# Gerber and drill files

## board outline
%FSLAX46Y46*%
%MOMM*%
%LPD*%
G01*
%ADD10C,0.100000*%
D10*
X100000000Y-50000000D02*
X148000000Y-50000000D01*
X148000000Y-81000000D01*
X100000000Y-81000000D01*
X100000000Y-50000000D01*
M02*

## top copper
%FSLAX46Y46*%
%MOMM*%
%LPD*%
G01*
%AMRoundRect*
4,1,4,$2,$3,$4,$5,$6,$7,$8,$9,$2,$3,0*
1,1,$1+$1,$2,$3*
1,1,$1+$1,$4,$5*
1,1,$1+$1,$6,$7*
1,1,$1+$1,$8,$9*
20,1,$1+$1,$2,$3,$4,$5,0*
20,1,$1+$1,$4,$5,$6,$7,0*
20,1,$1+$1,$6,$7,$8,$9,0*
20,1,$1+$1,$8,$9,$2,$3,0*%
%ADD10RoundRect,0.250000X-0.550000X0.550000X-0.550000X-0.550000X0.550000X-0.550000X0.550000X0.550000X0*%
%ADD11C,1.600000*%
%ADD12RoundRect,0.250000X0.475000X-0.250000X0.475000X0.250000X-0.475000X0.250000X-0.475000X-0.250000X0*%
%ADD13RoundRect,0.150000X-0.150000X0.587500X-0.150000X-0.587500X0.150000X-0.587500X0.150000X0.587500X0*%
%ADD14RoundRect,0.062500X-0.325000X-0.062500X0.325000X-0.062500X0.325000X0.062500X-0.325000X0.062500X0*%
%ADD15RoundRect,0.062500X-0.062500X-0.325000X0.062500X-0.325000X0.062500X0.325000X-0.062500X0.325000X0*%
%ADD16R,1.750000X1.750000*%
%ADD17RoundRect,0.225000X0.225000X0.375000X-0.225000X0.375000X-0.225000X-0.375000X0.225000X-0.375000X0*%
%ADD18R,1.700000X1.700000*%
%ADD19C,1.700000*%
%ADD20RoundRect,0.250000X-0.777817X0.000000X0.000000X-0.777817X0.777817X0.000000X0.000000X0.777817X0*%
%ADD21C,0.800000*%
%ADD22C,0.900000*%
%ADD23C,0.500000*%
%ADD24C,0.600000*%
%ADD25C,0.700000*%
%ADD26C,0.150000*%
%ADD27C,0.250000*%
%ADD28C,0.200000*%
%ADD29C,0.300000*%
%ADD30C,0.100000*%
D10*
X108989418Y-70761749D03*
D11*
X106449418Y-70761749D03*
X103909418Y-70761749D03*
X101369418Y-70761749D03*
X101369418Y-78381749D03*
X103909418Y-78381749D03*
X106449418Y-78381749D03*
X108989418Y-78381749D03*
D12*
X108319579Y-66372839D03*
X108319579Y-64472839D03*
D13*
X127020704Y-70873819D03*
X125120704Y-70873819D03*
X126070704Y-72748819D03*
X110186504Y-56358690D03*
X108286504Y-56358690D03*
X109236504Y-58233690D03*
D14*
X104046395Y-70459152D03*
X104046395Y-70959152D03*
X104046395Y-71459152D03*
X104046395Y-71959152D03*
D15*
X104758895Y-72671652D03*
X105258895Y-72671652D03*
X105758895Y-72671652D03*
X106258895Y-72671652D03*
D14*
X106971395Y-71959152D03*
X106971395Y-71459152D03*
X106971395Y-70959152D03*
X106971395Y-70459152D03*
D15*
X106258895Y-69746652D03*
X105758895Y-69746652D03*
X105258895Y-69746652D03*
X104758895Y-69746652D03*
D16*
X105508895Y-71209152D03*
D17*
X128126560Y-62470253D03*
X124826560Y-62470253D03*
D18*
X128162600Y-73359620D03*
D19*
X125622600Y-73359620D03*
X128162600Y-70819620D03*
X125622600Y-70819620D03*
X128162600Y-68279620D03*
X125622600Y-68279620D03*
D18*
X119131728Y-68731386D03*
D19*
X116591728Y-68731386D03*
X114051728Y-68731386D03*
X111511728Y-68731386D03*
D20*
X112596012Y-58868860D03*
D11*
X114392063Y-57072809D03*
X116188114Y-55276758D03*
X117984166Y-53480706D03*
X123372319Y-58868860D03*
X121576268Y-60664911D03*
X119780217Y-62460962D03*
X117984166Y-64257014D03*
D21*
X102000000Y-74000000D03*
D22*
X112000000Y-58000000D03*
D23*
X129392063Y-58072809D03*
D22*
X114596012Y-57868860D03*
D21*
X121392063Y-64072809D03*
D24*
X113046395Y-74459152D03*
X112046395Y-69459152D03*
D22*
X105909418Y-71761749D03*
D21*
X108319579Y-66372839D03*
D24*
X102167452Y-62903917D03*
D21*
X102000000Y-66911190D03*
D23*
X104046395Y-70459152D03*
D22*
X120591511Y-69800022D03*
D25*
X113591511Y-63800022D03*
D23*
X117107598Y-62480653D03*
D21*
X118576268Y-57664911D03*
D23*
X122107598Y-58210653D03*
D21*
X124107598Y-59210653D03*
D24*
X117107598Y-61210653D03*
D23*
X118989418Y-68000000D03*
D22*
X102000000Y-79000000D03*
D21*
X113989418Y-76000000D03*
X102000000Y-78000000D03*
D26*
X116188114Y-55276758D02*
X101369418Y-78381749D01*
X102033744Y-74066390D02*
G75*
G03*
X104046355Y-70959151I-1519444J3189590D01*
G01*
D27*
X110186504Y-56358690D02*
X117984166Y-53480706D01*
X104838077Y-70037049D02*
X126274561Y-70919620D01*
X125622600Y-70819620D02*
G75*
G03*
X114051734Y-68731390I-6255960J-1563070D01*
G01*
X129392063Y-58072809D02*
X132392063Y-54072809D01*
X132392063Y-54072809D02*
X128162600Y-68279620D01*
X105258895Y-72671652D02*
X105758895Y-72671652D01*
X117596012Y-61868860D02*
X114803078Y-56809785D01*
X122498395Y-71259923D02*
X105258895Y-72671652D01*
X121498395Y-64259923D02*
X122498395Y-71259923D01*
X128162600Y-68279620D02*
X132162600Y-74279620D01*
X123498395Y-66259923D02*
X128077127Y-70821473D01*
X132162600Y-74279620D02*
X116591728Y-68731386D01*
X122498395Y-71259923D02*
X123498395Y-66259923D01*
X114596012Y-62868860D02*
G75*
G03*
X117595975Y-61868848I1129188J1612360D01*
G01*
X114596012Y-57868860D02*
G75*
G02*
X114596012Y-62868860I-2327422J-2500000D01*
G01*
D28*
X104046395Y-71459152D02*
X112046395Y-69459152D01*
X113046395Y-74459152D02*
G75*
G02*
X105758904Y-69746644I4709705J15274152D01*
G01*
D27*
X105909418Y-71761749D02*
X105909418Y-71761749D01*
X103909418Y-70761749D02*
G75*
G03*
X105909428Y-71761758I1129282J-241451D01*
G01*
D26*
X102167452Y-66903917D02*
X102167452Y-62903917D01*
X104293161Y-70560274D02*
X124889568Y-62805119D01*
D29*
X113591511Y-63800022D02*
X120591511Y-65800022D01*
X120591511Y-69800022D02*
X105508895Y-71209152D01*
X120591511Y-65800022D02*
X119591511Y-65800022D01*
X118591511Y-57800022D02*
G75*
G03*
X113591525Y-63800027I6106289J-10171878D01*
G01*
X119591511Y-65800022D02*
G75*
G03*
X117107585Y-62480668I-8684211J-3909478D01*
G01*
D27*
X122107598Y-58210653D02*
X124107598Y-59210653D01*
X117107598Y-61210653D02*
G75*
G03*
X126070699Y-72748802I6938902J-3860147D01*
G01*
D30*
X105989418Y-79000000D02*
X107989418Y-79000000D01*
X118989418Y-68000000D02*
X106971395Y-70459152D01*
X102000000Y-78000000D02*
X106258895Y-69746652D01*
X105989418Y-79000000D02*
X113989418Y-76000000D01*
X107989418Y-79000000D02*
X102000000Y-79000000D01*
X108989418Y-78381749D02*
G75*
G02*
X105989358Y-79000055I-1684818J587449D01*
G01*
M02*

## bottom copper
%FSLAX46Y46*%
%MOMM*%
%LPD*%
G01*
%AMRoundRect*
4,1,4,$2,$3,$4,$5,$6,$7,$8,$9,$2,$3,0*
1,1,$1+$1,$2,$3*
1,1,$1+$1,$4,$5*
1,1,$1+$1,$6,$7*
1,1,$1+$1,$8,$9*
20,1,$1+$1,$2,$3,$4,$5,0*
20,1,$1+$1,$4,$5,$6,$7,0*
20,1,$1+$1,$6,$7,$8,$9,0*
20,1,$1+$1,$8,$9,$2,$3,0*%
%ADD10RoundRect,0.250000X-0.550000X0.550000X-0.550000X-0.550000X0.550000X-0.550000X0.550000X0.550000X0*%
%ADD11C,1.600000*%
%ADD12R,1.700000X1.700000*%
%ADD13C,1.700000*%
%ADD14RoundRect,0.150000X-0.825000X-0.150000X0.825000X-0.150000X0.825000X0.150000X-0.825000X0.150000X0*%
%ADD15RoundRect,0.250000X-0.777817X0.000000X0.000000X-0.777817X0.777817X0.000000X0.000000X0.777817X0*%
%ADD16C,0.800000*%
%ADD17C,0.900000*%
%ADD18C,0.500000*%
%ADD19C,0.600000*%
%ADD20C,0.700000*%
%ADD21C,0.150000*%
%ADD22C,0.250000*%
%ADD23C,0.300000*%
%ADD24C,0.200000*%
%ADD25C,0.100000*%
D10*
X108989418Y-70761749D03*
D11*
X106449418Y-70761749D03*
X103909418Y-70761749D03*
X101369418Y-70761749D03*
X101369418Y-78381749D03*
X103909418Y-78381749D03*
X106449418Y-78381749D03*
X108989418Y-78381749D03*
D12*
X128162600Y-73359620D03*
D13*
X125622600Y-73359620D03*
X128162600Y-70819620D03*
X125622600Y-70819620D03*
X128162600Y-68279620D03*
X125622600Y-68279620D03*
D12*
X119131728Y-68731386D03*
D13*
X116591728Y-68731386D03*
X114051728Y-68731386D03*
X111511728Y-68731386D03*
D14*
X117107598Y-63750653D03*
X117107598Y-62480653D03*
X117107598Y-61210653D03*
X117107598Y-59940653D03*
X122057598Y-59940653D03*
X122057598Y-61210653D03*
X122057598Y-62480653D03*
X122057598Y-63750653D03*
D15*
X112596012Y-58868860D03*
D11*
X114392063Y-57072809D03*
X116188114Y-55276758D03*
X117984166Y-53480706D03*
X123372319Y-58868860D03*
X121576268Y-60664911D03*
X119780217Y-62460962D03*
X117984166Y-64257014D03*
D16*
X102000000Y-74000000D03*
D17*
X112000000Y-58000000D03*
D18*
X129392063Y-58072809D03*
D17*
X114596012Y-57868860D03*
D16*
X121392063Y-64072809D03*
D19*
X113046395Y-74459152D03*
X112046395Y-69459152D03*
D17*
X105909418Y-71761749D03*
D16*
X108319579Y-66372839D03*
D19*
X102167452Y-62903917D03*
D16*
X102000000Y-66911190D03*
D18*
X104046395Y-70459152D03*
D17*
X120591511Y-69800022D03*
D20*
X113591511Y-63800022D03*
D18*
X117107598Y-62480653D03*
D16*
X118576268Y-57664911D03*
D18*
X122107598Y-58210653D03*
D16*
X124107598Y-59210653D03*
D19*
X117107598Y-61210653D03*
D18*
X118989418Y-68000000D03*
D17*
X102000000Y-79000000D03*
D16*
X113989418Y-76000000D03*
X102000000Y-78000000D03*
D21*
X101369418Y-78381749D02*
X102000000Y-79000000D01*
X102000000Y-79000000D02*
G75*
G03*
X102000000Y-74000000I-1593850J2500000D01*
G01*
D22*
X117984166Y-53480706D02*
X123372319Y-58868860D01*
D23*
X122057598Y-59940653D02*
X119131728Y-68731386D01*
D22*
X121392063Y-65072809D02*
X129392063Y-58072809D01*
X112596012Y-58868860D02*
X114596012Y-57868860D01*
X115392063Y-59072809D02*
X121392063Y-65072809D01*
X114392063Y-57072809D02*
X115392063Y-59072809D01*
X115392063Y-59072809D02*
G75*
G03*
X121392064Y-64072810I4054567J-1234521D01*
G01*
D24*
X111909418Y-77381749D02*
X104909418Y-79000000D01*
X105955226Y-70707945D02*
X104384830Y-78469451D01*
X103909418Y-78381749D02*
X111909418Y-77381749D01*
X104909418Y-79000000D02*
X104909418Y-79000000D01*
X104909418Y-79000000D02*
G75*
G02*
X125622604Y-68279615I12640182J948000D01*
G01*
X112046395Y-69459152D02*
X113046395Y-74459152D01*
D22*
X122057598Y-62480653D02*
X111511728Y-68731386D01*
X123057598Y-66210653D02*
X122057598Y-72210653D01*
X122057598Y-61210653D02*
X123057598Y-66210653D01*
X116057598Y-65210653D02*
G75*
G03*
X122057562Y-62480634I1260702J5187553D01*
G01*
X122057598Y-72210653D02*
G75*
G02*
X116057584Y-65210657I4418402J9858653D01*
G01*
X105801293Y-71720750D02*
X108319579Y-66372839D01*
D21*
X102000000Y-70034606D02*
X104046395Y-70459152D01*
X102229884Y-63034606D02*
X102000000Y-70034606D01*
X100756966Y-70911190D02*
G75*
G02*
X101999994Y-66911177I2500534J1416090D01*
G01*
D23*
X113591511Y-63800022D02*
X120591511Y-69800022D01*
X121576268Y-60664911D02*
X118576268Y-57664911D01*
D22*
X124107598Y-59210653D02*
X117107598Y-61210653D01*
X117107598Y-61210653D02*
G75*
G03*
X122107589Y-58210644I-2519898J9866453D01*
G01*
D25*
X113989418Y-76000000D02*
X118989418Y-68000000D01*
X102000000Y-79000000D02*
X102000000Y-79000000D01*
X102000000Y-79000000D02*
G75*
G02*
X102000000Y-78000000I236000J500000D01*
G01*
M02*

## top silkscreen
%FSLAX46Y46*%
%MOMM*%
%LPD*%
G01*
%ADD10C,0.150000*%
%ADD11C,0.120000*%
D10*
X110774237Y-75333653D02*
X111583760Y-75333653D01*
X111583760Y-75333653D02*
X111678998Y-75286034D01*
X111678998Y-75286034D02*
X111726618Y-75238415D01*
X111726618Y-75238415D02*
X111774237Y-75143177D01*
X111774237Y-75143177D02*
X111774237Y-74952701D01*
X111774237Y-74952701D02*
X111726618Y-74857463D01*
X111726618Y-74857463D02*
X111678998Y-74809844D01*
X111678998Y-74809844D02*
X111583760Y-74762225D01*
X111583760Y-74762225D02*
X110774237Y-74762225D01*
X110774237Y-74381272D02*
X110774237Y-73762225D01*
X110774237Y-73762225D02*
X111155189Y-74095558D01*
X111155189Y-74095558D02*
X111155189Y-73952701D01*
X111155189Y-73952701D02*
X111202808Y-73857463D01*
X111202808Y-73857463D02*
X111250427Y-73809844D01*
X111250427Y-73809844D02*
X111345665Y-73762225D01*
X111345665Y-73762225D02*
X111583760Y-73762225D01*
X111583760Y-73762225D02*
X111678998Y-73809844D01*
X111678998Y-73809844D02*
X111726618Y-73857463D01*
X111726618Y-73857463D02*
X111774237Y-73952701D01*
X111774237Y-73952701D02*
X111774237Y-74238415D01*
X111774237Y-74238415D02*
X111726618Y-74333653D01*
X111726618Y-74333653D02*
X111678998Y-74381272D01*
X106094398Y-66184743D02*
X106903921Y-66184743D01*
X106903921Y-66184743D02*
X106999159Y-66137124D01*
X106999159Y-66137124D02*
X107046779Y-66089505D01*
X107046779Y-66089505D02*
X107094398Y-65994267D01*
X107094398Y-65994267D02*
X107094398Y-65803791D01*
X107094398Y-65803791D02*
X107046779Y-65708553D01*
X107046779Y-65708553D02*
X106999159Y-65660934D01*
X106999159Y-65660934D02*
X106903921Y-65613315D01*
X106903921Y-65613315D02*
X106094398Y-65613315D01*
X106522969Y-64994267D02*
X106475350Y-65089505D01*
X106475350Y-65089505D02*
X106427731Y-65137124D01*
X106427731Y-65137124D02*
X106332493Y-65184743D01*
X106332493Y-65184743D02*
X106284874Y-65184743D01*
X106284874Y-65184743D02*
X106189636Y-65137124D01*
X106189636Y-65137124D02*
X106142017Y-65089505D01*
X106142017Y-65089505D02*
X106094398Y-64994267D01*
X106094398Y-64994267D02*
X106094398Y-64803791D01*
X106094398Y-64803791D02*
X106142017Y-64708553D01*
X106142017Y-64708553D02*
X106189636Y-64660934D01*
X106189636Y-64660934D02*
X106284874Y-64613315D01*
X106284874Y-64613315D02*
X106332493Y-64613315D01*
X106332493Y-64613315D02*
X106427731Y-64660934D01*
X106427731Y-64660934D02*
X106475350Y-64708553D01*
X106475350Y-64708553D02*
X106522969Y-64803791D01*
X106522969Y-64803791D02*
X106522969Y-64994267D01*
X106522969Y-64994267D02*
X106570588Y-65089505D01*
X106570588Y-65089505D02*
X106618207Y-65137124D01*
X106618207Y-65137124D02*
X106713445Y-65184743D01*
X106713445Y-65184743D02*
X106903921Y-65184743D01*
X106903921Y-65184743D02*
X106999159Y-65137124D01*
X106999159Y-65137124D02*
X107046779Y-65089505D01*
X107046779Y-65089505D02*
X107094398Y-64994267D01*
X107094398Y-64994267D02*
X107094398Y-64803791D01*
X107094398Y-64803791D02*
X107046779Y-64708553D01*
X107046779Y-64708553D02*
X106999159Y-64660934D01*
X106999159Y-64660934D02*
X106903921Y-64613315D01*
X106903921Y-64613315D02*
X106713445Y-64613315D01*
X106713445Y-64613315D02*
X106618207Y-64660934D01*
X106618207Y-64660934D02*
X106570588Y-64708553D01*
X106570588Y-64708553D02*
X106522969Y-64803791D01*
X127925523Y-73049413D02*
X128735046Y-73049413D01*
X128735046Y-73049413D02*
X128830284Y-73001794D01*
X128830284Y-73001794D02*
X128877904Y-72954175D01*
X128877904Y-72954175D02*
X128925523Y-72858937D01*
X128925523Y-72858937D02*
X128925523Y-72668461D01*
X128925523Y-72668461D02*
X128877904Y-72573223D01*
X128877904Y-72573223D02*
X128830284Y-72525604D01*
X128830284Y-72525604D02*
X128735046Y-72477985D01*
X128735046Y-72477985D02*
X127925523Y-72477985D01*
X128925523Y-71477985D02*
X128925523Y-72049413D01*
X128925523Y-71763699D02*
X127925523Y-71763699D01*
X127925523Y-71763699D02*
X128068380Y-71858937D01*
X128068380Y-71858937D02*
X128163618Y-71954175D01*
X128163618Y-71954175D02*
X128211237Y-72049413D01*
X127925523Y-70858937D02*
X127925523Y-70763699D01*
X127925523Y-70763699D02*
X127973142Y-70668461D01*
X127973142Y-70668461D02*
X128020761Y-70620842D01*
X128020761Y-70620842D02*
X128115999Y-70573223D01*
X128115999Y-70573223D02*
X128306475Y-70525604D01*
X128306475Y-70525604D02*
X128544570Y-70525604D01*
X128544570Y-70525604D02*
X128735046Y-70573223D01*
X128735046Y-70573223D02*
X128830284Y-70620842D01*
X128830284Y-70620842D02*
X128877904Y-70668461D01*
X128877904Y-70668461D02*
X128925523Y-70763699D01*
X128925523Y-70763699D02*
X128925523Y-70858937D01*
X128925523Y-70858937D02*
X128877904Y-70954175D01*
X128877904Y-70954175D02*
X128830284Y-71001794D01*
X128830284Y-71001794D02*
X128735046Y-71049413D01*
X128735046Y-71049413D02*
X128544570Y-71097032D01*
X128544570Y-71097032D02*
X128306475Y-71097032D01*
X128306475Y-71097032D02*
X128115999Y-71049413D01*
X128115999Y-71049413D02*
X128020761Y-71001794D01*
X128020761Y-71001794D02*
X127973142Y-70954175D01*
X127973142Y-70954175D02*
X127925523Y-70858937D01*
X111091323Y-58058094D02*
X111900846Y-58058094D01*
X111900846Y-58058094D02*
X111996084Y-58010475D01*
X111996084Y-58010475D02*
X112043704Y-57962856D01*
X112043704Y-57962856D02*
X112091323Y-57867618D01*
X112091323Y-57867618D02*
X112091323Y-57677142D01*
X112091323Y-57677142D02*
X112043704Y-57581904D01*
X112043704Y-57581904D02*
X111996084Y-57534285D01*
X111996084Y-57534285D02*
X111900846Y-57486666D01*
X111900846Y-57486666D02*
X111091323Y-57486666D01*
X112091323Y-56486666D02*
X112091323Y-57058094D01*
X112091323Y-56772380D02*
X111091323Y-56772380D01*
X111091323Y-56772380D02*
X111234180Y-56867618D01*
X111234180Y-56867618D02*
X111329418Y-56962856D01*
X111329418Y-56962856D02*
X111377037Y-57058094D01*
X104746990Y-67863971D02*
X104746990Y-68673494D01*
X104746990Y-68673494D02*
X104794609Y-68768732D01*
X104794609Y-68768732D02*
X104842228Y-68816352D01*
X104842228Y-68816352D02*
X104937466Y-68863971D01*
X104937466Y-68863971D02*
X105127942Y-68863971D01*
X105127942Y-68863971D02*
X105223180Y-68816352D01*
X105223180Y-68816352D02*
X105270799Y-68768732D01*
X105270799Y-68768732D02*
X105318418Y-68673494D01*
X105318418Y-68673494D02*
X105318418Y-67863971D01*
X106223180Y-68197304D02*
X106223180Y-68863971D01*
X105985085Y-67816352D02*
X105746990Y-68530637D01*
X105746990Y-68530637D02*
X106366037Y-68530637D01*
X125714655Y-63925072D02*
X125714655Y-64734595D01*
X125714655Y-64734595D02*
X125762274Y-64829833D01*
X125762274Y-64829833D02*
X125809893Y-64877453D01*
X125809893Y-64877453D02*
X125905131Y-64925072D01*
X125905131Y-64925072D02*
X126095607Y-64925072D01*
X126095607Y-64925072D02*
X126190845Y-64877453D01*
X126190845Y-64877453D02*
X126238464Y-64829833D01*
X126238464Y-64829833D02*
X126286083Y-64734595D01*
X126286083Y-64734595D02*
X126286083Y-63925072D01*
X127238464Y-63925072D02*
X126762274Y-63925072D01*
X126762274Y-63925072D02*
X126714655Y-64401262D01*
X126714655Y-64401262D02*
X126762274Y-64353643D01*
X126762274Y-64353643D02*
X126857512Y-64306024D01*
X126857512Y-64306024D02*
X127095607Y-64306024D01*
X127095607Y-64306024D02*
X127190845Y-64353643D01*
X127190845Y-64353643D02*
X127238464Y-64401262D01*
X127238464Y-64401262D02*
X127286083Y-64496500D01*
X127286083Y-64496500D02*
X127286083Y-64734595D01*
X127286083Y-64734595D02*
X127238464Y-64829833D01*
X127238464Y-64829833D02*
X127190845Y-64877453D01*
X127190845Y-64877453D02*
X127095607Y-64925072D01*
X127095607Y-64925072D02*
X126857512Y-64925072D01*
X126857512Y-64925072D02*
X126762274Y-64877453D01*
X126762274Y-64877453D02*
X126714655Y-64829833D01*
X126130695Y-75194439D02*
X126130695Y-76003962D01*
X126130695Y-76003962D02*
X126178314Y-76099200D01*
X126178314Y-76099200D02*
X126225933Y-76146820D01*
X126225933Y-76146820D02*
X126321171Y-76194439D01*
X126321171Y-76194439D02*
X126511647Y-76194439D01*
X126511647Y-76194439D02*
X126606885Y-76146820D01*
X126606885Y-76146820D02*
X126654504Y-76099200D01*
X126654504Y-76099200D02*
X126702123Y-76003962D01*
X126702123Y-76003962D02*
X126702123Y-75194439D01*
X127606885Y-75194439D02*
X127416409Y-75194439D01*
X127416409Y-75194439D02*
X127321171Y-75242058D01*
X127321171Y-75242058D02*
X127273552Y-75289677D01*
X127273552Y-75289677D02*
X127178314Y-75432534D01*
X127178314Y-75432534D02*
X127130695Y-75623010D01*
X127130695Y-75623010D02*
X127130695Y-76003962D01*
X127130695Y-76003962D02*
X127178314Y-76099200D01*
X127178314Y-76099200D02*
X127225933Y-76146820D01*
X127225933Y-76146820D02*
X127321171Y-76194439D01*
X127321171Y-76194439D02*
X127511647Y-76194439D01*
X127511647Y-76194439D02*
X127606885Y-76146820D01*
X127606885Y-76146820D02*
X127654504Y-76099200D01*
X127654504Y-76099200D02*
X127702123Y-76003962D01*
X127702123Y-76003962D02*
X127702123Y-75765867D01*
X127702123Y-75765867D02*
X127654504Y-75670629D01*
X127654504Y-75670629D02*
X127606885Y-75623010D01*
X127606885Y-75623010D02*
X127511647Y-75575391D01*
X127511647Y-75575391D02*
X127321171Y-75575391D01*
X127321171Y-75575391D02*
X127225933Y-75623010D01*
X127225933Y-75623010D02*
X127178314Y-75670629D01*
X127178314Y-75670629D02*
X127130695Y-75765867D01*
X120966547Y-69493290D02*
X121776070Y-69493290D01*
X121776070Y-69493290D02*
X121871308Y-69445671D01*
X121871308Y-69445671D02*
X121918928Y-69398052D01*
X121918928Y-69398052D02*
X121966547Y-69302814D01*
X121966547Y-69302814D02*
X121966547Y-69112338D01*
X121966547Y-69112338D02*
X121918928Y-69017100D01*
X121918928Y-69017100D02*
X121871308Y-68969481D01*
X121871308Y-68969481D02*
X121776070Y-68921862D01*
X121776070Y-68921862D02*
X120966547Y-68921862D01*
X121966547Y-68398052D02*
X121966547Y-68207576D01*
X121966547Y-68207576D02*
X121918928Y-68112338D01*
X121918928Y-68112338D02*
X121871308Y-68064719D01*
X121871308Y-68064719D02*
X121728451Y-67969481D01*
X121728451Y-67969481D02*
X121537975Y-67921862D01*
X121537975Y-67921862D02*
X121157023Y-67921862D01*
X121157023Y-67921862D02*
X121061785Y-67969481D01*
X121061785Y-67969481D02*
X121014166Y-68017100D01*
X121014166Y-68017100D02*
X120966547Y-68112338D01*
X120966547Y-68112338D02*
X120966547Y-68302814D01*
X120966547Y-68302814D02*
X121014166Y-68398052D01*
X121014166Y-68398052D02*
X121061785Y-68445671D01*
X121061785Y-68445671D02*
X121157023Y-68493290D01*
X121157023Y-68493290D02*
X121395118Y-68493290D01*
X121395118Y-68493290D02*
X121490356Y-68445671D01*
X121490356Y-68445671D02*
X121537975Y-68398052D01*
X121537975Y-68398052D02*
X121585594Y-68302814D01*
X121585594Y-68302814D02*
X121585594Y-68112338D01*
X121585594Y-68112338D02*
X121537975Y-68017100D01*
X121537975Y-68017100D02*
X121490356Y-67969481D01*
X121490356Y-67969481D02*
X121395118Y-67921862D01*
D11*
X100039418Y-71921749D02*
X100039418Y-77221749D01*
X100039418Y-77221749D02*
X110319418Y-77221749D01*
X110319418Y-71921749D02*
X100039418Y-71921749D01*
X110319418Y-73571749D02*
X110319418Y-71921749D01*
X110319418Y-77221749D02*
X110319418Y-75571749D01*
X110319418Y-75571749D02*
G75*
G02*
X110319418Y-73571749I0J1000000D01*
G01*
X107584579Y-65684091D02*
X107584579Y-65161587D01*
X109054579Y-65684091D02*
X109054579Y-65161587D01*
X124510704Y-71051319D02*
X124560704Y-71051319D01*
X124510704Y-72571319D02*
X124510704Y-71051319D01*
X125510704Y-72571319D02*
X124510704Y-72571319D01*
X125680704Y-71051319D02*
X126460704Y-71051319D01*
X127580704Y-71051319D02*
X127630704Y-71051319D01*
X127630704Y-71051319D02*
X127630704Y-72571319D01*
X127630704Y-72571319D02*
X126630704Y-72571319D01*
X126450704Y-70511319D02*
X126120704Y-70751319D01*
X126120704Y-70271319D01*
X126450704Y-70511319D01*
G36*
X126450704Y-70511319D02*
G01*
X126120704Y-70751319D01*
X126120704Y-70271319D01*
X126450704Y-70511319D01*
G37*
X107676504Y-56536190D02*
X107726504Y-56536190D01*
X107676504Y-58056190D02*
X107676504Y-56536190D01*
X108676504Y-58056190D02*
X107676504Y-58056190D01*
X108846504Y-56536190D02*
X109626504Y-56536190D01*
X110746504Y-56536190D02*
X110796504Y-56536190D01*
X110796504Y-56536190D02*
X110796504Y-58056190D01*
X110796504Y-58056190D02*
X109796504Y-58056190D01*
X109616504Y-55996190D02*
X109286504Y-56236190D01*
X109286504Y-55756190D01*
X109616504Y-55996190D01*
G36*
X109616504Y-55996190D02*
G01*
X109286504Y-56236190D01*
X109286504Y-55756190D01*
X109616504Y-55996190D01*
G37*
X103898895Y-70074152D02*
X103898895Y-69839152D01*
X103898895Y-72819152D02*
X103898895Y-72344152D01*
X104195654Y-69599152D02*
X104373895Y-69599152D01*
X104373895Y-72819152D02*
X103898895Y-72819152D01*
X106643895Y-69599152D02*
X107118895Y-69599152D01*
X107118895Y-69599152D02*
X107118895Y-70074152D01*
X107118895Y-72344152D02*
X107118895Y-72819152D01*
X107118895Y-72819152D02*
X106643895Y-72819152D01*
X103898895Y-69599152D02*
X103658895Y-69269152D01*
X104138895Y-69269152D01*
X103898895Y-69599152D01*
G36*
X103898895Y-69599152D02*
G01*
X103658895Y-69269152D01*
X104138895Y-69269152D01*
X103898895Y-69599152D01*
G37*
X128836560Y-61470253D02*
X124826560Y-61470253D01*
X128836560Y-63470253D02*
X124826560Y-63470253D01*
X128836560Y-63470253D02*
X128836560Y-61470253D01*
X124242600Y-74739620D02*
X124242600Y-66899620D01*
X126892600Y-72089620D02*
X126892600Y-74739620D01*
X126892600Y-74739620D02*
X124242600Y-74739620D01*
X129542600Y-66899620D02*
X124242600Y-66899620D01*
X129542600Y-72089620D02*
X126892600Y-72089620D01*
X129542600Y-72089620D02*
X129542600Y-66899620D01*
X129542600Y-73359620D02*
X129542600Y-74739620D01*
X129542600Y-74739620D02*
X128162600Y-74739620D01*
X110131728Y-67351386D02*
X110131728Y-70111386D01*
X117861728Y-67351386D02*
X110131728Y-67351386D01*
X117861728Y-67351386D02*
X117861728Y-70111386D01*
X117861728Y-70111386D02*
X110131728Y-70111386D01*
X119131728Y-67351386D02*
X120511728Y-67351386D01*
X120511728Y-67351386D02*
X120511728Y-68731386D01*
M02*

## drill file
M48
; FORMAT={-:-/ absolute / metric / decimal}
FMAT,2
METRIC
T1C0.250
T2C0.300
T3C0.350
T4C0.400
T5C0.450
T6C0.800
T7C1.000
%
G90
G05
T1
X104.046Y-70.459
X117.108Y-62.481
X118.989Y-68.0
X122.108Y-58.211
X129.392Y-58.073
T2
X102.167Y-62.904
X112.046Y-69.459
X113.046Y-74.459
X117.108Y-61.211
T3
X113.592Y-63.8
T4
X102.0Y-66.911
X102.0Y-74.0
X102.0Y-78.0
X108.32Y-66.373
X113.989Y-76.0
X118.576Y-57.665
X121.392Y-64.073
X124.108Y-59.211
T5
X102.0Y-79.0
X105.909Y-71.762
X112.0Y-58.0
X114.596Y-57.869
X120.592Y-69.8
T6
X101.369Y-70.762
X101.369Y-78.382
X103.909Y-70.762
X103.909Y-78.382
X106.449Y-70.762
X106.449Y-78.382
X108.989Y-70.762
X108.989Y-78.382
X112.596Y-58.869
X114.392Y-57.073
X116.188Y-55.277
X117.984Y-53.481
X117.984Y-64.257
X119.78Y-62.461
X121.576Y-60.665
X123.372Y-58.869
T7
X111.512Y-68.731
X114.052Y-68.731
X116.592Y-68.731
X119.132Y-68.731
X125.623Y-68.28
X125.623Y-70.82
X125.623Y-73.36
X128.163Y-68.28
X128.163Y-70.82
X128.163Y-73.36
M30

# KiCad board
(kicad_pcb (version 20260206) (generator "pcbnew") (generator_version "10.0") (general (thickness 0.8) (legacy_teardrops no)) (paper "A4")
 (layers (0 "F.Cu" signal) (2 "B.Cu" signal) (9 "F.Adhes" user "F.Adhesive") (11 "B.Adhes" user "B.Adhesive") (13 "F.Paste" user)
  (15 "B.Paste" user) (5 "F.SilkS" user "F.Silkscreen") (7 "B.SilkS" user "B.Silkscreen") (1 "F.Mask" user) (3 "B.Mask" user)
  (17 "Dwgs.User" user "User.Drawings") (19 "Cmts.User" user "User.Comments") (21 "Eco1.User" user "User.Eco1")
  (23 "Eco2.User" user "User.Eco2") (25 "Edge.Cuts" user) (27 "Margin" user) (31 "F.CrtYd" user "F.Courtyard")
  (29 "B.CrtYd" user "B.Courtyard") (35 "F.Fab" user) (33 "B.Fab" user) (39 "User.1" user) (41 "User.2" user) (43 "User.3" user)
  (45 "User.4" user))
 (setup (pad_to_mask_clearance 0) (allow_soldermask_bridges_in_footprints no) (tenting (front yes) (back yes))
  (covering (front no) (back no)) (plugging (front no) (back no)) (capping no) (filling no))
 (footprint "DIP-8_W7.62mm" (layer "F.Cu") (at 108.989418 70.761749 -90)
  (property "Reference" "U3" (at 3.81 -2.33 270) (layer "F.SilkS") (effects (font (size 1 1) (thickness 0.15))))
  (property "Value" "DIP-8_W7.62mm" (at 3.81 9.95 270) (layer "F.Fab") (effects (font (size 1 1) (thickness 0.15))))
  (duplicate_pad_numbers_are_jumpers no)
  (fp_line (start 1.16 8.95) (end 6.46 8.95) (stroke (width 0.12) (type solid)) (layer "F.SilkS"))
  (fp_line (start 6.46 8.95) (end 6.46 -1.33) (stroke (width 0.12) (type solid)) (layer "F.SilkS"))
  (fp_line (start 1.16 -1.33) (end 1.16 8.95) (stroke (width 0.12) (type solid)) (layer "F.SilkS"))
  (fp_line (start 2.81 -1.33) (end 1.16 -1.33) (stroke (width 0.12) (type solid)) (layer "F.SilkS"))
  (fp_line (start 6.46 -1.33) (end 4.81 -1.33) (stroke (width 0.12) (type solid)) (layer "F.SilkS"))
  (fp_arc (start 4.81 -1.33) (mid 3.81 -0.33) (end 2.81 -1.33) (stroke (width 0.12) (type solid)) (layer "F.SilkS"))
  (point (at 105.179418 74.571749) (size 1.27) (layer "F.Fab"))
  (pad "1" thru_hole roundrect (at 0 0 270) (size 1.6 1.6) (drill 0.8) (layers "*.Cu" "*.Mask") (remove_unused_layers no)
   (roundrect_rratio 0.15625))
  (pad "2" thru_hole circle (at 0 2.54 270) (size 1.6 1.6) (drill 0.8) (layers "*.Cu" "*.Mask") (remove_unused_layers no) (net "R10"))
  (pad "3" thru_hole circle (at 0 5.08 270) (size 1.6 1.6) (drill 0.8) (layers "*.Cu" "*.Mask") (remove_unused_layers no) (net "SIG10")
   (die_length 0.3))
  (pad "4" thru_hole circle (at 0 7.62 270) (size 1.6 1.6) (drill 0.8) (layers "*.Cu" "*.Mask") (remove_unused_layers no)
   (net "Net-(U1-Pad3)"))
  (pad "5" thru_hole circle (at 7.62 7.62 270) (size 1.6 1.6) (drill 0.8) (layers "*.Cu" "*.Mask") (remove_unused_layers no)
   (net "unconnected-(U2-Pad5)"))
  (pad "6" thru_hole circle (at 7.62 5.08 270) (size 1.6 1.6) (drill 0.8) (layers "*.Cu" "*.Mask") (remove_unused_layers no) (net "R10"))
  (pad "7" thru_hole circle (at 7.62 2.54 270) (size 1.6 1.6) (drill 0.8) (layers "*.Cu" "*.Mask") (remove_unused_layers no))
  (pad "8" thru_hole circle (at 7.62 0 270) (size 1.6 1.6) (drill 0.8) (layers "*.Cu" "*.Mask") (remove_unused_layers no) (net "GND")))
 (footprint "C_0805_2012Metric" (layer "F.Cu") (at 108.319579 65.422839 90)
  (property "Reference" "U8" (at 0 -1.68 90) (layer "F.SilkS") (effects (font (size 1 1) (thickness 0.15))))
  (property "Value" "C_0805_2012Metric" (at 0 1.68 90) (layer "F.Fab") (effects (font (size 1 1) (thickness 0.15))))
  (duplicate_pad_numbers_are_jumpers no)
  (fp_line (start -0.261252 -0.735) (end 0.261252 -0.735) (stroke (width 0.12) (type solid)) (layer "F.SilkS"))
  (fp_line (start -0.261252 0.735) (end 0.261252 0.735) (stroke (width 0.12) (type solid)) (layer "F.SilkS"))
  (pad "1" smd roundrect (at -0.95 0 90) (size 1 1.45) (layers "F.Cu" "F.Mask" "F.Paste") (roundrect_rratio 0.25) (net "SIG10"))
  (pad "2" smd roundrect (at 0.95 0 90) (size 1 1.45) (layers "F.Cu" "F.Mask" "F.Paste") (roundrect_rratio 0.25)))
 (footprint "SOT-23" (layer "F.Cu") (at 126.070704 71.811319 -90)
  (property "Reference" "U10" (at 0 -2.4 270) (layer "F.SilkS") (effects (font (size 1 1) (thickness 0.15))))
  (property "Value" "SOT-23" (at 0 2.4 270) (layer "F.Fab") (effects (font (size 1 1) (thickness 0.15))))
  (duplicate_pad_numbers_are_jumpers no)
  (fp_line (start -0.76 1.56) (end -0.76 1.51) (stroke (width 0.12) (type solid)) (layer "F.SilkS"))
  (fp_line (start 0.76 1.56) (end -0.76 1.56) (stroke (width 0.12) (type solid)) (layer "F.SilkS"))
  (fp_line (start 0.76 0.56) (end 0.76 1.56) (stroke (width 0.12) (type solid)) (layer "F.SilkS"))
  (fp_line (start -0.76 0.39) (end -0.76 -0.39) (stroke (width 0.12) (type solid)) (layer "F.SilkS"))
  (fp_line (start -0.76 -1.51) (end -0.76 -1.56) (stroke (width 0.12) (type solid)) (layer "F.SilkS"))
  (fp_line (start -0.76 -1.56) (end 0.76 -1.56) (stroke (width 0.12) (type solid)) (layer "F.SilkS"))
  (fp_line (start 0.76 -1.56) (end 0.76 -0.56) (stroke (width 0.12) (type solid)) (layer "F.SilkS"))
  (fp_poly (pts (xy -1.3 -0.38) (xy -1.06 -0.05) (xy -1.54 -0.05)) (stroke (width 0.12) (type solid)) (fill yes) (layer "F.SilkS"))
  (pad "1" smd roundrect (at -0.9375 -0.95 270) (size 1.475 0.6) (layers "F.Cu" "F.Mask" "F.Paste") (roundrect_rratio 0.25)
   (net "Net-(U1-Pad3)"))
  (pad "2" smd roundrect (at -0.9375 0.95 270) (size 1.475 0.6) (layers "F.Cu" "F.Mask" "F.Paste") (roundrect_rratio 0.25) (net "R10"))
  (pad "3" smd roundrect (at 0.9375 0 270) (size 1.475 0.6) (layers "F.Cu" "F.Mask" "F.Paste") (roundrect_rratio 0.25) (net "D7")
   (die_length 2.7)))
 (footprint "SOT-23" (layer "F.Cu") (at 109.236504 57.29619 -90)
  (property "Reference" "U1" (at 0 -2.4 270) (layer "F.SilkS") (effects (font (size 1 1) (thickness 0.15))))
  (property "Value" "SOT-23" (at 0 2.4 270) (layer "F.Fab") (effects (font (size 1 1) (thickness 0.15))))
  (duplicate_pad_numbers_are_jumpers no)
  (fp_line (start -0.76 1.56) (end -0.76 1.51) (stroke (width 0.12) (type solid)) (layer "F.SilkS"))
  (fp_line (start 0.76 1.56) (end -0.76 1.56) (stroke (width 0.12) (type solid)) (layer "F.SilkS"))
  (fp_line (start 0.76 0.56) (end 0.76 1.56) (stroke (width 0.12) (type solid)) (layer "F.SilkS"))
  (fp_line (start -0.76 0.39) (end -0.76 -0.39) (stroke (width 0.12) (type solid)) (layer "F.SilkS"))
  (fp_line (start -0.76 -1.51) (end -0.76 -1.56) (stroke (width 0.12) (type solid)) (layer "F.SilkS"))
  (fp_line (start -0.76 -1.56) (end 0.76 -1.56) (stroke (width 0.12) (type solid)) (layer "F.SilkS"))
  (fp_line (start 0.76 -1.56) (end 0.76 -0.56) (stroke (width 0.12) (type solid)) (layer "F.SilkS"))
  (fp_poly (pts (xy -1.3 -0.38) (xy -1.06 -0.05) (xy -1.54 -0.05)) (stroke (width 0.12) (type solid)) (fill yes) (layer "F.SilkS"))
  (pad "1" smd roundrect (at -0.9375 -0.95 270) (size 1.475 0.6) (layers "F.Cu" "F.Mask" "F.Paste") (roundrect_rratio 0.25) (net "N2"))
  (pad "2" smd roundrect (at -0.9375 0.95 270) (size 1.475 0.6) (layers "F.Cu" "F.Mask" "F.Paste") (roundrect_rratio 0.25))
  (pad "3" smd roundrect (at 0.9375 0 270) (size 1.475 0.6) (layers "F.Cu" "F.Mask" "F.Paste") (roundrect_rratio 0.25) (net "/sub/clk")
   (die_length 2.5)))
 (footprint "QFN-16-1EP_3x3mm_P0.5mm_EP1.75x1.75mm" (layer "F.Cu") (at 105.508895 71.209152)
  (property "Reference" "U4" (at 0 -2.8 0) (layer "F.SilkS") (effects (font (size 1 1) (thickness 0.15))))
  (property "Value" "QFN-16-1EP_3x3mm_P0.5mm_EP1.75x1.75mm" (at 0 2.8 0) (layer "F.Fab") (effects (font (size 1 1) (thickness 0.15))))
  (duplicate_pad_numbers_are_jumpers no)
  (fp_line (start -1.61 -1.135) (end -1.61 -1.37) (stroke (width 0.12) (type solid)) (layer "F.SilkS"))
  (fp_line (start -1.61 1.61) (end -1.61 1.135) (stroke (width 0.12) (type solid)) (layer "F.SilkS"))
  (fp_line (start -1.313241 -1.61) (end -1.135 -1.61) (stroke (width 0.12) (type solid)) (layer "F.SilkS"))
  (fp_line (start -1.135 1.61) (end -1.61 1.61) (stroke (width 0.12) (type solid)) (layer "F.SilkS"))
  (fp_line (start 1.135 -1.61) (end 1.61 -1.61) (stroke (width 0.12) (type solid)) (layer "F.SilkS"))
  (fp_line (start 1.61 -1.61) (end 1.61 -1.135) (stroke (width 0.12) (type solid)) (layer "F.SilkS"))
  (fp_line (start 1.61 1.135) (end 1.61 1.61) (stroke (width 0.12) (type solid)) (layer "F.SilkS"))
  (fp_line (start 1.61 1.61) (end 1.135 1.61) (stroke (width 0.12) (type solid)) (layer "F.SilkS"))
  (fp_poly (pts (xy -1.61 -1.61) (xy -1.85 -1.94) (xy -1.37 -1.94)) (stroke (width 0.12) (type solid)) (fill yes) (layer "F.SilkS"))
  (pad "" smd roundrect (at -0.44 -0.44) (size 0.71 0.71) (layers "F.Paste") (roundrect_rratio 0.25))
  (pad "" smd roundrect (at -0.44 0.44) (size 0.71 0.71) (layers "F.Paste") (roundrect_rratio 0.25) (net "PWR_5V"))
  (pad "" smd roundrect (at 0.44 -0.44) (size 0.71 0.71) (layers "F.Paste") (roundrect_rratio 0.25))
  (pad "" smd roundrect (at 0.44 0.44) (size 0.71 0.71) (layers "F.Paste") (roundrect_rratio 0.25))
  (pad "1" smd roundrect (at -1.4625 -0.75) (size 0.775 0.25) (layers "F.Cu" "F.Mask" "F.Paste") (roundrect_rratio 0.25)
   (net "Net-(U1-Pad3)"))
  (pad "2" smd roundrect (at -1.4625 -0.25) (size 0.775 0.25) (layers "F.Cu" "F.Mask" "F.Paste") (roundrect_rratio 0.25)
   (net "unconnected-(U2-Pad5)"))
  (pad "3" smd roundrect (at -1.4625 0.25) (size 0.775 0.25) (layers "F.Cu" "F.Mask" "F.Paste") (roundrect_rratio 0.25) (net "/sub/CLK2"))
  (pad "4" smd roundrect (at -1.4625 0.75) (size 0.775 0.25) (layers "F.Cu" "F.Mask" "F.Paste") (roundrect_rratio 0.25))
  (pad "5" smd roundrect (at -0.75 1.4625) (size 0.25 0.775) (layers "F.Cu" "F.Mask" "F.Paste") (roundrect_rratio 0.25) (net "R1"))
  (pad "6" smd roundrect (at -0.25 1.4625) (size 0.25 0.775) (layers "F.Cu" "F.Mask" "F.Paste") (roundrect_rratio 0.25) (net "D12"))
  (pad "7" smd roundrect (at 0.25 1.4625) (size 0.25 0.775) (layers "F.Cu" "F.Mask" "F.Paste") (roundrect_rratio 0.25) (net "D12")
   (die_length 3.3))
  (pad "8" smd roundrect (at 0.75 1.4625) (size 0.25 0.775) (layers "F.Cu" "F.Mask" "F.Paste") (roundrect_rratio 0.25))
  (pad "9" smd roundrect (at 1.4625 0.75) (size 0.775 0.25) (layers "F.Cu" "F.Mask" "F.Paste") (roundrect_rratio 0.25))
  (pad "10" smd roundrect (at 1.4625 0.25) (size 0.775 0.25) (layers "F.Cu" "F.Mask" "F.Paste") (roundrect_rratio 0.25))
  (pad "11" smd roundrect (at 1.4625 -0.25) (size 0.775 0.25) (layers "F.Cu" "F.Mask" "F.Paste") (roundrect_rratio 0.25))
  (pad "12" smd roundrect (at 1.4625 -0.75) (size 0.775 0.25) (layers "F.Cu" "F.Mask" "F.Paste") (roundrect_rratio 0.25) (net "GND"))
  (pad "13" smd roundrect (at 0.75 -1.4625) (size 0.25 0.775) (layers "F.Cu" "F.Mask" "F.Paste") (roundrect_rratio 0.25) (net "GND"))
  (pad "14" smd roundrect (at 0.25 -1.4625) (size 0.25 0.775) (layers "F.Cu" "F.Mask" "F.Paste") (roundrect_rratio 0.25) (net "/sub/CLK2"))
  (pad "15" smd roundrect (at -0.25 -1.4625) (size 0.25 0.775) (layers "F.Cu" "F.Mask" "F.Paste") (roundrect_rratio 0.25))
  (pad "16" smd roundrect (at -0.75 -1.4625) (size 0.25 0.775) (layers "F.Cu" "F.Mask" "F.Paste") (roundrect_rratio 0.25) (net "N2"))
  (pad "17" smd rect (at 0 0) (size 1.75 1.75) (layers "F.Cu" "F.Mask") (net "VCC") (zone_connect 2)))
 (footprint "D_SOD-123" (layer "F.Cu") (at 126.47656 62.470253 180)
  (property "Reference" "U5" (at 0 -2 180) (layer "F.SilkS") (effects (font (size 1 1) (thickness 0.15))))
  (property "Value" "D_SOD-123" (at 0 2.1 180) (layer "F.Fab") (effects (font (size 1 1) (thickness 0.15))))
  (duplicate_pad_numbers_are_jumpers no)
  (fp_line (start -2.36 1) (end 1.65 1) (stroke (width 0.12) (type solid)) (layer "F.SilkS"))
  (fp_line (start -2.36 -1) (end 1.65 -1) (stroke (width 0.12) (type solid)) (layer "F.SilkS"))
  (fp_line (start -2.36 -1) (end -2.36 1) (stroke (width 0.12) (type solid)) (layer "F.SilkS"))
  (pad "1" smd roundrect (at -1.65 0 180) (size 0.9 1.2) (layers "F.Cu" "F.Mask" "F.Paste") (roundrect_rratio 0.25))
  (pad "2" smd roundrect (at 1.65 0 180) (size 0.9 1.2) (layers "F.Cu" "F.Mask" "F.Paste") (roundrect_rratio 0.25) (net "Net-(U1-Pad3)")))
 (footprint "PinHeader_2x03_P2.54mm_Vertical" (layer "F.Cu") (at 128.1626 73.35962 180)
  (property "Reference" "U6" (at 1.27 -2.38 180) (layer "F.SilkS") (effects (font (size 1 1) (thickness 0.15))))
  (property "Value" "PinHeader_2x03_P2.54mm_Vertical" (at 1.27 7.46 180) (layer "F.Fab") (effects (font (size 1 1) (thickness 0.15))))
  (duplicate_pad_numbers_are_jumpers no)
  (fp_line (start 3.92 -1.38) (end 3.92 6.46) (stroke (width 0.12) (type solid)) (layer "F.SilkS"))
  (fp_line (start 1.27 1.27) (end 1.27 -1.38) (stroke (width 0.12) (type solid)) (layer "F.SilkS"))
  (fp_line (start 1.27 -1.38) (end 3.92 -1.38) (stroke (width 0.12) (type solid)) (layer "F.SilkS"))
  (fp_line (start -1.38 6.46) (end 3.92 6.46) (stroke (width 0.12) (type solid)) (layer "F.SilkS"))
  (fp_line (start -1.38 1.27) (end 1.27 1.27) (stroke (width 0.12) (type solid)) (layer "F.SilkS"))
  (fp_line (start -1.38 1.27) (end -1.38 6.46) (stroke (width 0.12) (type solid)) (layer "F.SilkS"))
  (fp_line (start -1.38 0) (end -1.38 -1.38) (stroke (width 0.12) (type solid)) (layer "F.SilkS"))
  (fp_line (start -1.38 -1.38) (end 0 -1.38) (stroke (width 0.12) (type solid)) (layer "F.SilkS"))
  (pad "1" thru_hole rect (at 0 0 180) (size 1.7 1.7) (drill 1) (layers "*.Cu" "*.Mask") (remove_unused_layers no) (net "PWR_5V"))
  (pad "2" thru_hole circle (at 2.54 0 180) (size 1.7 1.7) (drill 1) (layers "*.Cu" "*.Mask") (remove_unused_layers no))
  (pad "3" thru_hole circle (at 0 2.54 180) (size 1.7 1.7) (drill 1) (layers "*.Cu" "*.Mask") (remove_unused_layers no) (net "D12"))
  (pad "4" thru_hole circle (at 2.54 2.54 180) (size 1.7 1.7) (drill 1) (layers "*.Cu" "*.Mask") (remove_unused_layers no) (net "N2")
   (die_length 0.1))
  (pad "5" thru_hole circle (at 0 5.08 180) (size 1.7 1.7) (drill 1) (layers "*.Cu" "*.Mask") (remove_unused_layers no) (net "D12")
   (die_length 2.7))
  (pad "6" thru_hole circle (at 2.54 5.08 180) (size 1.7 1.7) (drill 1) (layers "*.Cu" "*.Mask") (remove_unused_layers no) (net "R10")
   (die_length 0.6)))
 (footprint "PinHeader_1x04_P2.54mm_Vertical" (layer "F.Cu") (at 119.131728 68.731386 -90)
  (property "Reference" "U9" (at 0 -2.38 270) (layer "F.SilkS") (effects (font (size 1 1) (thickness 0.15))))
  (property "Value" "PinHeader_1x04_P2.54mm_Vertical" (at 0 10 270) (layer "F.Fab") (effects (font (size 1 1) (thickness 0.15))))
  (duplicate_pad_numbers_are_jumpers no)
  (fp_line (start -1.38 9) (end 1.38 9) (stroke (width 0.12) (type solid)) (layer "F.SilkS"))
  (fp_line (start -1.38 1.27) (end -1.38 9) (stroke (width 0.12) (type solid)) (layer "F.SilkS"))
  (fp_line (start -1.38 1.27) (end 1.38 1.27) (stroke (width 0.12) (type solid)) (layer "F.SilkS"))
  (fp_line (start 1.38 1.27) (end 1.38 9) (stroke (width 0.12) (type solid)) (layer "F.SilkS"))
  (fp_line (start -1.38 0) (end -1.38 -1.38) (stroke (width 0.12) (type solid)) (layer "F.SilkS"))
  (fp_line (start -1.38 -1.38) (end 0 -1.38) (stroke (width 0.12) (type solid)) (layer "F.SilkS"))
  (pad "1" thru_hole rect (at 0 0 270) (size 1.7 1.7) (drill 1) (layers "*.Cu" "*.Mask") (remove_unused_layers no) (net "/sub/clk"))
  (pad "2" thru_hole circle (at 0 2.54 270) (size 1.7 1.7) (drill 1) (layers "*.Cu" "*.Mask") (remove_unused_layers no) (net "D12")
   (die_length 4.4))
  (pad "3" thru_hole circle (at 0 5.08 270) (size 1.7 1.7) (drill 1) (layers "*.Cu" "*.Mask") (remove_unused_layers no) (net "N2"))
  (pad "4" thru_hole circle (at 0 7.62 270) (size 1.7 1.7) (drill 1) (layers "*.Cu" "*.Mask") (remove_unused_layers no) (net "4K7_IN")))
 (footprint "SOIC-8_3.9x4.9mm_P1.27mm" (layer "B.Cu") (at 119.582598 61.845653)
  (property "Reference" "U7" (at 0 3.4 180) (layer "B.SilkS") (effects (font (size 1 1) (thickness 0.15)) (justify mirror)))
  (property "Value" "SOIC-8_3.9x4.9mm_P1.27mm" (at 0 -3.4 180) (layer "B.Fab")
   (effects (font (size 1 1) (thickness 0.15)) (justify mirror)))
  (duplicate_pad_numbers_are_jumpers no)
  (pad "1" smd roundrect (at -2.475 1.905) (size 1.95 0.6) (layers "B.Cu" "B.Mask" "B.Paste") (roundrect_rratio 0.25))
  (pad "2" smd roundrect (at -2.475 0.635) (size 1.95 0.6) (layers "B.Cu" "B.Mask" "B.Paste") (roundrect_rratio 0.25) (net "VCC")
   (die_length 1.7))
  (pad "3" smd roundrect (at -2.475 -0.635) (size 1.95 0.6) (layers "B.Cu" "B.Mask" "B.Paste") (roundrect_rratio 0.25) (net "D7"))
  (pad "4" smd roundrect (at -2.475 -1.905) (size 1.95 0.6) (layers "B.Cu" "B.Mask" "B.Paste") (roundrect_rratio 0.25) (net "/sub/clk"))
  (pad "5" smd roundrect (at 2.475 -1.905) (size 1.95 0.6) (layers "B.Cu" "B.Mask" "B.Paste") (roundrect_rratio 0.25) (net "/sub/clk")
   (die_length 1.6))
  (pad "6" smd roundrect (at 2.475 -0.635) (size 1.95 0.6) (layers "B.Cu" "B.Mask" "B.Paste") (roundrect_rratio 0.25) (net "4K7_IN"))
  (pad "7" smd roundrect (at 2.475 0.635) (size 1.95 0.6) (layers "B.Cu" "B.Mask" "B.Paste") (roundrect_rratio 0.25) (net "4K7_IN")
   (die_length 3.2))
  (pad "8" smd roundrect (at 2.475 1.905) (size 1.95 0.6) (layers "B.Cu" "B.Mask" "B.Paste") (roundrect_rratio 0.25)))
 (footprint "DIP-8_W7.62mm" (layer "B.Cu") (at 112.596012 58.86886 -45)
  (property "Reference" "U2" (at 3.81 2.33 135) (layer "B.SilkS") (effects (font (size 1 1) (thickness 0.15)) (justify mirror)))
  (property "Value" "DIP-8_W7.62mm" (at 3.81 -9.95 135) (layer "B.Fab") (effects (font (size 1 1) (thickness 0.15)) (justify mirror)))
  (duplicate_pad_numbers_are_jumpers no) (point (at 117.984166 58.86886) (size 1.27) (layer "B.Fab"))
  (pad "1" thru_hole roundrect (at 0 0 315) (size 1.6 1.6) (drill 0.8) (layers "*.Cu" "*.Mask") (remove_unused_layers no)
   (roundrect_rratio 0.15625) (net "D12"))
  (pad "2" thru_hole circle (at 0 -2.54 315) (size 1.6 1.6) (drill 0.8) (layers "*.Cu" "*.Mask") (remove_unused_layers no) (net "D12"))
  (pad "3" thru_hole circle (at 0 -5.079999 315) (size 1.6 1.6) (drill 0.8) (layers "*.Cu" "*.Mask") (remove_unused_layers no)
   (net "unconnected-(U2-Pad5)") (die_length 4.5))
  (pad "4" thru_hole circle (at 0 -7.62 315) (size 1.6 1.6) (drill 0.8) (layers "*.Cu" "*.Mask") (remove_unused_layers no) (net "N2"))
  (pad "5" thru_hole circle (at 7.62 -7.62 315) (size 1.6 1.6) (drill 0.8) (layers "*.Cu" "*.Mask") (remove_unused_layers no) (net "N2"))
  (pad "6" thru_hole circle (at 7.62 -5.08 315) (size 1.6 1.6) (drill 0.8) (layers "*.Cu" "*.Mask") (remove_unused_layers no) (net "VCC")
   (die_length 1.5))
  (pad "7" thru_hole circle (at 7.62 -2.54 315) (size 1.6 1.6) (drill 0.8) (layers "*.Cu" "*.Mask") (remove_unused_layers no)
   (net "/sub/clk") (die_length 1.6))
  (pad "8" thru_hole circle (at 7.62 0 315) (size 1.6 1.6) (drill 0.8) (layers "*.Cu" "*.Mask") (remove_unused_layers no)))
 (gr_rect (start 100 50) (end 148 81) (stroke (width 0.1) (type default)) (fill no) (layer "Edge.Cuts"))
 (segment (start 116.188114 55.276758) (end 101.369418 78.381749) (width 0.15) (layer "F.Cu") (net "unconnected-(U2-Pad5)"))
 (via (at 102 74) (size 0.8) (drill 0.4) (layers "F.Cu" "B.Cu") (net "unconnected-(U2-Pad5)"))
 (arc (start 102.033744 74.06639) (mid 103.479646 72.797498) (end 104.046395 70.959152) (width 0.15) (layer "F.Cu")
  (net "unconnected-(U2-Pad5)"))
 (segment (start 101.369418 78.381749) (end 102 79) (width 0.15) (layer "B.Cu") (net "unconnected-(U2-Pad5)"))
 (arc (start 102 79) (mid 103.371004 76.5) (end 102 74) (width 0.15) (layer "B.Cu") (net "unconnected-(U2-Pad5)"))
 (segment (start 110.186504 56.35869) (end 117.984166 53.480706) (width 0.25) (layer "F.Cu") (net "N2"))
 (segment (start 104.838077 70.037049) (end 126.274561 70.91962) (width 0.25) (layer "F.Cu") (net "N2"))
 (via (at 112 58) (size 0.9) (drill 0.45) (layers "F.Cu" "B.Cu") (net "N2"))
 (arc (start 125.6226 70.81962) (mid 120.511877 66.036926) (end 114.051728 68.731386) (width 0.25) (layer "F.Cu") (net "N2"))
 (segment (start 117.984166 53.480706) (end 123.372319 58.86886) (width 0.25) (layer "B.Cu") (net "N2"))
 (segment (start 122.057598 59.940653) (end 119.131728 68.731386) (width 0.3) (layer "B.Cu") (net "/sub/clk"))
 (segment (start 129.392063 58.072809) (end 132.392063 54.072809) (width 0.25) (layer "F.Cu") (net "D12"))
 (segment (start 132.392063 54.072809) (end 128.1626 68.27962) (width 0.25) (layer "F.Cu") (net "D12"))
 (segment (start 105.258895 72.671652) (end 105.758895 72.671652) (width 0.25) (layer "F.Cu") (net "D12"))
 (segment (start 117.596012 61.86886) (end 114.803078 56.809785) (width 0.25) (layer "F.Cu") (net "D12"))
 (segment (start 122.498395 71.259923) (end 105.258895 72.671652) (width 0.25) (layer "F.Cu") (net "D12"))
 (segment (start 121.498395 64.259923) (end 122.498395 71.259923) (width 0.25) (layer "F.Cu") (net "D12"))
 (segment (start 128.1626 68.27962) (end 132.1626 74.27962) (width 0.25) (layer "F.Cu") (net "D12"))
 (segment (start 123.498395 66.259923) (end 128.077127 70.821473) (width 0.25) (layer "F.Cu") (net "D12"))
 (segment (start 132.1626 74.27962) (end 116.591728 68.731386) (width 0.25) (layer "F.Cu") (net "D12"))
 (segment (start 122.498395 71.259923) (end 123.498395 66.259923) (width 0.25) (layer "F.Cu") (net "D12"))
 (via (at 129.392063 58.072809) (size 0.5) (drill 0.25) (layers "F.Cu" "B.Cu") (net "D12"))
 (via (at 114.596012 57.86886) (size 0.9) (drill 0.45) (layers "F.Cu" "B.Cu") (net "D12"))
 (via (at 121.392063 64.072809) (size 0.8) (drill 0.4) (layers "F.Cu" "B.Cu") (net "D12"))
 (arc (start 114.596012 62.86886) (mid 116.347708 63.123949) (end 117.596012 61.86886) (width 0.25) (layer "F.Cu") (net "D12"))
 (arc (start 114.596012 57.86886) (mid 115.684274 60.36886) (end 114.596012 62.86886) (width 0.25) (layer "F.Cu") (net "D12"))
 (segment (start 121.392063 65.072809) (end 129.392063 58.072809) (width 0.25) (layer "B.Cu") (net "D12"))
 (segment (start 112.596012 58.86886) (end 114.596012 57.86886) (width 0.25) (layer "B.Cu") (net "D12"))
 (segment (start 115.392063 59.072809) (end 121.392063 65.072809) (width 0.25) (layer "B.Cu") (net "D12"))
 (segment (start 114.392063 57.072809) (end 115.392063 59.072809) (width 0.25) (layer "B.Cu") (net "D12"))
 (arc (start 115.392063 59.072809) (mid 116.733308 63.563314) (end 121.392063 64.072809) (width 0.25) (layer "B.Cu") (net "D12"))
 (segment (start 111.909418 77.381749) (end 104.909418 79) (width 0.2) (layer "B.Cu") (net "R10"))
 (segment (start 105.955226 70.707945) (end 104.38483 78.469451) (width 0.2) (layer "B.Cu") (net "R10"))
 (segment (start 103.909418 78.381749) (end 111.909418 77.381749) (width 0.2) (layer "B.Cu") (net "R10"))
 (segment (start 104.909418 79) (end 104.909418 79) (width 0.2) (layer "B.Cu") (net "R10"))
 (arc (start 104.909418 79) (mid 111.72324 66.794716) (end 125.6226 68.27962) (width 0.2) (layer "B.Cu") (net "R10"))
 (segment (start 104.046395 71.459152) (end 112.046395 69.459152) (width 0.2) (layer "F.Cu") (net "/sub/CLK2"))
 (via (at 113.046395 74.459152) (size 0.6) (drill 0.3) (layers "F.Cu" "B.Cu") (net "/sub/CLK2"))
 (via (at 112.046395 69.459152) (size 0.6) (drill 0.3) (layers "F.Cu" "B.Cu") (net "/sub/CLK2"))
 (arc (start 113.046395 74.459152) (mid 109.076691 72.606963) (end 105.758895 69.746652) (width 0.2) (layer "F.Cu") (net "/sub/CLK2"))
 (segment (start 112.046395 69.459152) (end 113.046395 74.459152) (width 0.2) (layer "B.Cu") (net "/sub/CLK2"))
 (segment (start 122.057598 62.480653) (end 111.511728 68.731386) (width 0.25) (layer "B.Cu") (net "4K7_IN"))
 (segment (start 123.057598 66.210653) (end 122.057598 72.210653) (width 0.25) (layer "B.Cu") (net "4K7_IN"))
 (segment (start 122.057598 61.210653) (end 123.057598 66.210653) (width 0.25) (layer "B.Cu") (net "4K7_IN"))
 (arc (start 116.057598 65.210653) (mid 119.529277 64.88231) (end 122.057598 62.480653) (width 0.25) (layer "B.Cu") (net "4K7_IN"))
 (arc (start 122.057598 72.210653) (mid 118.273399 69.382823) (end 116.057598 65.210653) (width 0.25) (layer "B.Cu") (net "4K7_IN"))
 (segment (start 105.909418 71.761749) (end 105.909418 71.761749) (width 0.25) (layer "F.Cu") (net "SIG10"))
 (via (at 105.909418 71.761749) (size 0.9) (drill 0.45) (layers "F.Cu" "B.Cu") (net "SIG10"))
 (via (at 108.319579 66.372839) (size 0.8) (drill 0.4) (layers "F.Cu" "B.Cu") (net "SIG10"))
 (arc (start 103.909418 70.761749) (mid 104.522233 72.036117) (end 105.909418 71.761749) (width 0.25) (layer "F.Cu") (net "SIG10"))
 (segment (start 105.801293 71.72075) (end 108.319579 66.372839) (width 0.25) (layer "B.Cu") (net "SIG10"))
 (segment (start 102.167452 66.903917) (end 102.167452 62.903917) (width 0.15) (layer "F.Cu") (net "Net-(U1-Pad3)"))
 (segment (start 104.293161 70.560274) (end 124.889568 62.805119) (width 0.15) (layer "F.Cu") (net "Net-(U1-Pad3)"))
 (via (at 102.167452 62.903917) (size 0.6) (drill 0.3) (layers "F.Cu" "B.Cu") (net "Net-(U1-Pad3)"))
 (via (at 102 66.91119) (size 0.8) (drill 0.4) (layers "F.Cu" "B.Cu") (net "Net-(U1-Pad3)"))
 (via (at 104.046395 70.459152) (size 0.5) (drill 0.25) (layers "F.Cu" "B.Cu") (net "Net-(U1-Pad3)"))
 (segment (start 102 70.034606) (end 104.046395 70.459152) (width 0.15) (layer "B.Cu") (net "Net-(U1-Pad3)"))
 (segment (start 102.229884 63.034606) (end 102 70.034606) (width 0.15) (layer "B.Cu") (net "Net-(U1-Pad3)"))
 (arc (start 100.756966 70.91119) (mid 100.513273 68.642318) (end 102 66.91119) (width 0.15) (layer "B.Cu") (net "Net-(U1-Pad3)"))
 (segment (start 113.591511 63.800022) (end 120.591511 65.800022) (width 0.3) (layer "F.Cu") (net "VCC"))
 (segment (start 120.591511 69.800022) (end 105.508895 71.209152) (width 0.3) (layer "F.Cu") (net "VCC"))
 (segment (start 120.591511 65.800022) (end 119.591511 65.800022) (width 0.3) (layer "F.Cu") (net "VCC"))
 (via (at 120.591511 69.800022) (size 0.9) (drill 0.45) (layers "F.Cu" "B.Cu") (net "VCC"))
 (via (at 113.591511 63.800022) (size 0.7) (drill 0.35) (layers "F.Cu" "B.Cu") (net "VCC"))
 (via (at 117.107598 62.480653) (size 0.5) (drill 0.25) (layers "F.Cu" "B.Cu") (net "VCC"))
 (via (at 118.576268 57.664911) (size 0.8) (drill 0.4) (layers "F.Cu" "B.Cu") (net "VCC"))
 (arc (start 118.591511 57.800022) (mid 115.583622 60.376781) (end 113.591511 63.800022) (width 0.3) (layer "F.Cu") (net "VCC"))
 (arc (start 119.591511 65.800022) (mid 118.53237 64.003534) (end 117.107598 62.480653) (width 0.3) (layer "F.Cu") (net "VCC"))
 (segment (start 113.591511 63.800022) (end 120.591511 69.800022) (width 0.3) (layer "B.Cu") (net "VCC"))
 (segment (start 121.576268 60.664911) (end 118.576268 57.664911) (width 0.3) (layer "B.Cu") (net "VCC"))
 (segment (start 122.107598 58.210653) (end 124.107598 59.210653) (width 0.25) (layer "F.Cu") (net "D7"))
 (via (at 122.107598 58.210653) (size 0.5) (drill 0.25) (layers "F.Cu" "B.Cu") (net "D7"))
 (via (at 124.107598 59.210653) (size 0.8) (drill 0.4) (layers "F.Cu" "B.Cu") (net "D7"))
 (via (at 117.107598 61.210653) (size 0.6) (drill 0.3) (layers "F.Cu" "B.Cu") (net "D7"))
 (arc (start 117.107598 61.210653) (mid 117.775869 69.941978) (end 126.070704 72.748819) (width 0.25) (layer "F.Cu") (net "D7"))
 (segment (start 124.107598 59.210653) (end 117.107598 61.210653) (width 0.25) (layer "B.Cu") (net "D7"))
 (arc (start 117.107598 61.210653) (mid 119.826915 60.076182) (end 122.107598 58.210653) (width 0.25) (layer "B.Cu") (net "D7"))
 (segment (start 105.989418 79) (end 107.989418 79) (width 0.1) (layer "F.Cu") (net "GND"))
 (segment (start 118.989418 68) (end 106.971395 70.459152) (width 0.1) (layer "F.Cu") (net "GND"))
 (segment (start 102 78) (end 106.258895 69.746652) (width 0.1) (layer "F.Cu") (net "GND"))
 (segment (start 105.989418 79) (end 113.989418 76) (width 0.1) (layer "F.Cu") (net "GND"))
 (segment (start 107.989418 79) (end 102 79) (width 0.1) (layer "F.Cu") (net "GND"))
 (via (at 118.989418 68) (size 0.5) (drill 0.25) (layers "F.Cu" "B.Cu") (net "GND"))
 (via (at 102 79) (size 0.9) (drill 0.45) (layers "F.Cu" "B.Cu") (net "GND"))
 (via (at 113.989418 76) (size 0.8) (drill 0.4) (layers "F.Cu" "B.Cu") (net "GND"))
 (via (at 102 78) (size 0.8) (drill 0.4) (layers "F.Cu" "B.Cu") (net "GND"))
 (arc (start 108.989418 78.381749) (mid 107.664785 79.541828) (end 105.989418 79) (width 0.1) (layer "F.Cu") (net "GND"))
 (segment (start 113.989418 76) (end 118.989418 68) (width 0.1) (layer "B.Cu") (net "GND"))
 (segment (start 102 79) (end 102 79) (width 0.1) (layer "B.Cu") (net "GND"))
 (arc (start 102 79) (mid 101.68312 78.5) (end 102 78) (width 0.1) (layer "B.Cu") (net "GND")))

